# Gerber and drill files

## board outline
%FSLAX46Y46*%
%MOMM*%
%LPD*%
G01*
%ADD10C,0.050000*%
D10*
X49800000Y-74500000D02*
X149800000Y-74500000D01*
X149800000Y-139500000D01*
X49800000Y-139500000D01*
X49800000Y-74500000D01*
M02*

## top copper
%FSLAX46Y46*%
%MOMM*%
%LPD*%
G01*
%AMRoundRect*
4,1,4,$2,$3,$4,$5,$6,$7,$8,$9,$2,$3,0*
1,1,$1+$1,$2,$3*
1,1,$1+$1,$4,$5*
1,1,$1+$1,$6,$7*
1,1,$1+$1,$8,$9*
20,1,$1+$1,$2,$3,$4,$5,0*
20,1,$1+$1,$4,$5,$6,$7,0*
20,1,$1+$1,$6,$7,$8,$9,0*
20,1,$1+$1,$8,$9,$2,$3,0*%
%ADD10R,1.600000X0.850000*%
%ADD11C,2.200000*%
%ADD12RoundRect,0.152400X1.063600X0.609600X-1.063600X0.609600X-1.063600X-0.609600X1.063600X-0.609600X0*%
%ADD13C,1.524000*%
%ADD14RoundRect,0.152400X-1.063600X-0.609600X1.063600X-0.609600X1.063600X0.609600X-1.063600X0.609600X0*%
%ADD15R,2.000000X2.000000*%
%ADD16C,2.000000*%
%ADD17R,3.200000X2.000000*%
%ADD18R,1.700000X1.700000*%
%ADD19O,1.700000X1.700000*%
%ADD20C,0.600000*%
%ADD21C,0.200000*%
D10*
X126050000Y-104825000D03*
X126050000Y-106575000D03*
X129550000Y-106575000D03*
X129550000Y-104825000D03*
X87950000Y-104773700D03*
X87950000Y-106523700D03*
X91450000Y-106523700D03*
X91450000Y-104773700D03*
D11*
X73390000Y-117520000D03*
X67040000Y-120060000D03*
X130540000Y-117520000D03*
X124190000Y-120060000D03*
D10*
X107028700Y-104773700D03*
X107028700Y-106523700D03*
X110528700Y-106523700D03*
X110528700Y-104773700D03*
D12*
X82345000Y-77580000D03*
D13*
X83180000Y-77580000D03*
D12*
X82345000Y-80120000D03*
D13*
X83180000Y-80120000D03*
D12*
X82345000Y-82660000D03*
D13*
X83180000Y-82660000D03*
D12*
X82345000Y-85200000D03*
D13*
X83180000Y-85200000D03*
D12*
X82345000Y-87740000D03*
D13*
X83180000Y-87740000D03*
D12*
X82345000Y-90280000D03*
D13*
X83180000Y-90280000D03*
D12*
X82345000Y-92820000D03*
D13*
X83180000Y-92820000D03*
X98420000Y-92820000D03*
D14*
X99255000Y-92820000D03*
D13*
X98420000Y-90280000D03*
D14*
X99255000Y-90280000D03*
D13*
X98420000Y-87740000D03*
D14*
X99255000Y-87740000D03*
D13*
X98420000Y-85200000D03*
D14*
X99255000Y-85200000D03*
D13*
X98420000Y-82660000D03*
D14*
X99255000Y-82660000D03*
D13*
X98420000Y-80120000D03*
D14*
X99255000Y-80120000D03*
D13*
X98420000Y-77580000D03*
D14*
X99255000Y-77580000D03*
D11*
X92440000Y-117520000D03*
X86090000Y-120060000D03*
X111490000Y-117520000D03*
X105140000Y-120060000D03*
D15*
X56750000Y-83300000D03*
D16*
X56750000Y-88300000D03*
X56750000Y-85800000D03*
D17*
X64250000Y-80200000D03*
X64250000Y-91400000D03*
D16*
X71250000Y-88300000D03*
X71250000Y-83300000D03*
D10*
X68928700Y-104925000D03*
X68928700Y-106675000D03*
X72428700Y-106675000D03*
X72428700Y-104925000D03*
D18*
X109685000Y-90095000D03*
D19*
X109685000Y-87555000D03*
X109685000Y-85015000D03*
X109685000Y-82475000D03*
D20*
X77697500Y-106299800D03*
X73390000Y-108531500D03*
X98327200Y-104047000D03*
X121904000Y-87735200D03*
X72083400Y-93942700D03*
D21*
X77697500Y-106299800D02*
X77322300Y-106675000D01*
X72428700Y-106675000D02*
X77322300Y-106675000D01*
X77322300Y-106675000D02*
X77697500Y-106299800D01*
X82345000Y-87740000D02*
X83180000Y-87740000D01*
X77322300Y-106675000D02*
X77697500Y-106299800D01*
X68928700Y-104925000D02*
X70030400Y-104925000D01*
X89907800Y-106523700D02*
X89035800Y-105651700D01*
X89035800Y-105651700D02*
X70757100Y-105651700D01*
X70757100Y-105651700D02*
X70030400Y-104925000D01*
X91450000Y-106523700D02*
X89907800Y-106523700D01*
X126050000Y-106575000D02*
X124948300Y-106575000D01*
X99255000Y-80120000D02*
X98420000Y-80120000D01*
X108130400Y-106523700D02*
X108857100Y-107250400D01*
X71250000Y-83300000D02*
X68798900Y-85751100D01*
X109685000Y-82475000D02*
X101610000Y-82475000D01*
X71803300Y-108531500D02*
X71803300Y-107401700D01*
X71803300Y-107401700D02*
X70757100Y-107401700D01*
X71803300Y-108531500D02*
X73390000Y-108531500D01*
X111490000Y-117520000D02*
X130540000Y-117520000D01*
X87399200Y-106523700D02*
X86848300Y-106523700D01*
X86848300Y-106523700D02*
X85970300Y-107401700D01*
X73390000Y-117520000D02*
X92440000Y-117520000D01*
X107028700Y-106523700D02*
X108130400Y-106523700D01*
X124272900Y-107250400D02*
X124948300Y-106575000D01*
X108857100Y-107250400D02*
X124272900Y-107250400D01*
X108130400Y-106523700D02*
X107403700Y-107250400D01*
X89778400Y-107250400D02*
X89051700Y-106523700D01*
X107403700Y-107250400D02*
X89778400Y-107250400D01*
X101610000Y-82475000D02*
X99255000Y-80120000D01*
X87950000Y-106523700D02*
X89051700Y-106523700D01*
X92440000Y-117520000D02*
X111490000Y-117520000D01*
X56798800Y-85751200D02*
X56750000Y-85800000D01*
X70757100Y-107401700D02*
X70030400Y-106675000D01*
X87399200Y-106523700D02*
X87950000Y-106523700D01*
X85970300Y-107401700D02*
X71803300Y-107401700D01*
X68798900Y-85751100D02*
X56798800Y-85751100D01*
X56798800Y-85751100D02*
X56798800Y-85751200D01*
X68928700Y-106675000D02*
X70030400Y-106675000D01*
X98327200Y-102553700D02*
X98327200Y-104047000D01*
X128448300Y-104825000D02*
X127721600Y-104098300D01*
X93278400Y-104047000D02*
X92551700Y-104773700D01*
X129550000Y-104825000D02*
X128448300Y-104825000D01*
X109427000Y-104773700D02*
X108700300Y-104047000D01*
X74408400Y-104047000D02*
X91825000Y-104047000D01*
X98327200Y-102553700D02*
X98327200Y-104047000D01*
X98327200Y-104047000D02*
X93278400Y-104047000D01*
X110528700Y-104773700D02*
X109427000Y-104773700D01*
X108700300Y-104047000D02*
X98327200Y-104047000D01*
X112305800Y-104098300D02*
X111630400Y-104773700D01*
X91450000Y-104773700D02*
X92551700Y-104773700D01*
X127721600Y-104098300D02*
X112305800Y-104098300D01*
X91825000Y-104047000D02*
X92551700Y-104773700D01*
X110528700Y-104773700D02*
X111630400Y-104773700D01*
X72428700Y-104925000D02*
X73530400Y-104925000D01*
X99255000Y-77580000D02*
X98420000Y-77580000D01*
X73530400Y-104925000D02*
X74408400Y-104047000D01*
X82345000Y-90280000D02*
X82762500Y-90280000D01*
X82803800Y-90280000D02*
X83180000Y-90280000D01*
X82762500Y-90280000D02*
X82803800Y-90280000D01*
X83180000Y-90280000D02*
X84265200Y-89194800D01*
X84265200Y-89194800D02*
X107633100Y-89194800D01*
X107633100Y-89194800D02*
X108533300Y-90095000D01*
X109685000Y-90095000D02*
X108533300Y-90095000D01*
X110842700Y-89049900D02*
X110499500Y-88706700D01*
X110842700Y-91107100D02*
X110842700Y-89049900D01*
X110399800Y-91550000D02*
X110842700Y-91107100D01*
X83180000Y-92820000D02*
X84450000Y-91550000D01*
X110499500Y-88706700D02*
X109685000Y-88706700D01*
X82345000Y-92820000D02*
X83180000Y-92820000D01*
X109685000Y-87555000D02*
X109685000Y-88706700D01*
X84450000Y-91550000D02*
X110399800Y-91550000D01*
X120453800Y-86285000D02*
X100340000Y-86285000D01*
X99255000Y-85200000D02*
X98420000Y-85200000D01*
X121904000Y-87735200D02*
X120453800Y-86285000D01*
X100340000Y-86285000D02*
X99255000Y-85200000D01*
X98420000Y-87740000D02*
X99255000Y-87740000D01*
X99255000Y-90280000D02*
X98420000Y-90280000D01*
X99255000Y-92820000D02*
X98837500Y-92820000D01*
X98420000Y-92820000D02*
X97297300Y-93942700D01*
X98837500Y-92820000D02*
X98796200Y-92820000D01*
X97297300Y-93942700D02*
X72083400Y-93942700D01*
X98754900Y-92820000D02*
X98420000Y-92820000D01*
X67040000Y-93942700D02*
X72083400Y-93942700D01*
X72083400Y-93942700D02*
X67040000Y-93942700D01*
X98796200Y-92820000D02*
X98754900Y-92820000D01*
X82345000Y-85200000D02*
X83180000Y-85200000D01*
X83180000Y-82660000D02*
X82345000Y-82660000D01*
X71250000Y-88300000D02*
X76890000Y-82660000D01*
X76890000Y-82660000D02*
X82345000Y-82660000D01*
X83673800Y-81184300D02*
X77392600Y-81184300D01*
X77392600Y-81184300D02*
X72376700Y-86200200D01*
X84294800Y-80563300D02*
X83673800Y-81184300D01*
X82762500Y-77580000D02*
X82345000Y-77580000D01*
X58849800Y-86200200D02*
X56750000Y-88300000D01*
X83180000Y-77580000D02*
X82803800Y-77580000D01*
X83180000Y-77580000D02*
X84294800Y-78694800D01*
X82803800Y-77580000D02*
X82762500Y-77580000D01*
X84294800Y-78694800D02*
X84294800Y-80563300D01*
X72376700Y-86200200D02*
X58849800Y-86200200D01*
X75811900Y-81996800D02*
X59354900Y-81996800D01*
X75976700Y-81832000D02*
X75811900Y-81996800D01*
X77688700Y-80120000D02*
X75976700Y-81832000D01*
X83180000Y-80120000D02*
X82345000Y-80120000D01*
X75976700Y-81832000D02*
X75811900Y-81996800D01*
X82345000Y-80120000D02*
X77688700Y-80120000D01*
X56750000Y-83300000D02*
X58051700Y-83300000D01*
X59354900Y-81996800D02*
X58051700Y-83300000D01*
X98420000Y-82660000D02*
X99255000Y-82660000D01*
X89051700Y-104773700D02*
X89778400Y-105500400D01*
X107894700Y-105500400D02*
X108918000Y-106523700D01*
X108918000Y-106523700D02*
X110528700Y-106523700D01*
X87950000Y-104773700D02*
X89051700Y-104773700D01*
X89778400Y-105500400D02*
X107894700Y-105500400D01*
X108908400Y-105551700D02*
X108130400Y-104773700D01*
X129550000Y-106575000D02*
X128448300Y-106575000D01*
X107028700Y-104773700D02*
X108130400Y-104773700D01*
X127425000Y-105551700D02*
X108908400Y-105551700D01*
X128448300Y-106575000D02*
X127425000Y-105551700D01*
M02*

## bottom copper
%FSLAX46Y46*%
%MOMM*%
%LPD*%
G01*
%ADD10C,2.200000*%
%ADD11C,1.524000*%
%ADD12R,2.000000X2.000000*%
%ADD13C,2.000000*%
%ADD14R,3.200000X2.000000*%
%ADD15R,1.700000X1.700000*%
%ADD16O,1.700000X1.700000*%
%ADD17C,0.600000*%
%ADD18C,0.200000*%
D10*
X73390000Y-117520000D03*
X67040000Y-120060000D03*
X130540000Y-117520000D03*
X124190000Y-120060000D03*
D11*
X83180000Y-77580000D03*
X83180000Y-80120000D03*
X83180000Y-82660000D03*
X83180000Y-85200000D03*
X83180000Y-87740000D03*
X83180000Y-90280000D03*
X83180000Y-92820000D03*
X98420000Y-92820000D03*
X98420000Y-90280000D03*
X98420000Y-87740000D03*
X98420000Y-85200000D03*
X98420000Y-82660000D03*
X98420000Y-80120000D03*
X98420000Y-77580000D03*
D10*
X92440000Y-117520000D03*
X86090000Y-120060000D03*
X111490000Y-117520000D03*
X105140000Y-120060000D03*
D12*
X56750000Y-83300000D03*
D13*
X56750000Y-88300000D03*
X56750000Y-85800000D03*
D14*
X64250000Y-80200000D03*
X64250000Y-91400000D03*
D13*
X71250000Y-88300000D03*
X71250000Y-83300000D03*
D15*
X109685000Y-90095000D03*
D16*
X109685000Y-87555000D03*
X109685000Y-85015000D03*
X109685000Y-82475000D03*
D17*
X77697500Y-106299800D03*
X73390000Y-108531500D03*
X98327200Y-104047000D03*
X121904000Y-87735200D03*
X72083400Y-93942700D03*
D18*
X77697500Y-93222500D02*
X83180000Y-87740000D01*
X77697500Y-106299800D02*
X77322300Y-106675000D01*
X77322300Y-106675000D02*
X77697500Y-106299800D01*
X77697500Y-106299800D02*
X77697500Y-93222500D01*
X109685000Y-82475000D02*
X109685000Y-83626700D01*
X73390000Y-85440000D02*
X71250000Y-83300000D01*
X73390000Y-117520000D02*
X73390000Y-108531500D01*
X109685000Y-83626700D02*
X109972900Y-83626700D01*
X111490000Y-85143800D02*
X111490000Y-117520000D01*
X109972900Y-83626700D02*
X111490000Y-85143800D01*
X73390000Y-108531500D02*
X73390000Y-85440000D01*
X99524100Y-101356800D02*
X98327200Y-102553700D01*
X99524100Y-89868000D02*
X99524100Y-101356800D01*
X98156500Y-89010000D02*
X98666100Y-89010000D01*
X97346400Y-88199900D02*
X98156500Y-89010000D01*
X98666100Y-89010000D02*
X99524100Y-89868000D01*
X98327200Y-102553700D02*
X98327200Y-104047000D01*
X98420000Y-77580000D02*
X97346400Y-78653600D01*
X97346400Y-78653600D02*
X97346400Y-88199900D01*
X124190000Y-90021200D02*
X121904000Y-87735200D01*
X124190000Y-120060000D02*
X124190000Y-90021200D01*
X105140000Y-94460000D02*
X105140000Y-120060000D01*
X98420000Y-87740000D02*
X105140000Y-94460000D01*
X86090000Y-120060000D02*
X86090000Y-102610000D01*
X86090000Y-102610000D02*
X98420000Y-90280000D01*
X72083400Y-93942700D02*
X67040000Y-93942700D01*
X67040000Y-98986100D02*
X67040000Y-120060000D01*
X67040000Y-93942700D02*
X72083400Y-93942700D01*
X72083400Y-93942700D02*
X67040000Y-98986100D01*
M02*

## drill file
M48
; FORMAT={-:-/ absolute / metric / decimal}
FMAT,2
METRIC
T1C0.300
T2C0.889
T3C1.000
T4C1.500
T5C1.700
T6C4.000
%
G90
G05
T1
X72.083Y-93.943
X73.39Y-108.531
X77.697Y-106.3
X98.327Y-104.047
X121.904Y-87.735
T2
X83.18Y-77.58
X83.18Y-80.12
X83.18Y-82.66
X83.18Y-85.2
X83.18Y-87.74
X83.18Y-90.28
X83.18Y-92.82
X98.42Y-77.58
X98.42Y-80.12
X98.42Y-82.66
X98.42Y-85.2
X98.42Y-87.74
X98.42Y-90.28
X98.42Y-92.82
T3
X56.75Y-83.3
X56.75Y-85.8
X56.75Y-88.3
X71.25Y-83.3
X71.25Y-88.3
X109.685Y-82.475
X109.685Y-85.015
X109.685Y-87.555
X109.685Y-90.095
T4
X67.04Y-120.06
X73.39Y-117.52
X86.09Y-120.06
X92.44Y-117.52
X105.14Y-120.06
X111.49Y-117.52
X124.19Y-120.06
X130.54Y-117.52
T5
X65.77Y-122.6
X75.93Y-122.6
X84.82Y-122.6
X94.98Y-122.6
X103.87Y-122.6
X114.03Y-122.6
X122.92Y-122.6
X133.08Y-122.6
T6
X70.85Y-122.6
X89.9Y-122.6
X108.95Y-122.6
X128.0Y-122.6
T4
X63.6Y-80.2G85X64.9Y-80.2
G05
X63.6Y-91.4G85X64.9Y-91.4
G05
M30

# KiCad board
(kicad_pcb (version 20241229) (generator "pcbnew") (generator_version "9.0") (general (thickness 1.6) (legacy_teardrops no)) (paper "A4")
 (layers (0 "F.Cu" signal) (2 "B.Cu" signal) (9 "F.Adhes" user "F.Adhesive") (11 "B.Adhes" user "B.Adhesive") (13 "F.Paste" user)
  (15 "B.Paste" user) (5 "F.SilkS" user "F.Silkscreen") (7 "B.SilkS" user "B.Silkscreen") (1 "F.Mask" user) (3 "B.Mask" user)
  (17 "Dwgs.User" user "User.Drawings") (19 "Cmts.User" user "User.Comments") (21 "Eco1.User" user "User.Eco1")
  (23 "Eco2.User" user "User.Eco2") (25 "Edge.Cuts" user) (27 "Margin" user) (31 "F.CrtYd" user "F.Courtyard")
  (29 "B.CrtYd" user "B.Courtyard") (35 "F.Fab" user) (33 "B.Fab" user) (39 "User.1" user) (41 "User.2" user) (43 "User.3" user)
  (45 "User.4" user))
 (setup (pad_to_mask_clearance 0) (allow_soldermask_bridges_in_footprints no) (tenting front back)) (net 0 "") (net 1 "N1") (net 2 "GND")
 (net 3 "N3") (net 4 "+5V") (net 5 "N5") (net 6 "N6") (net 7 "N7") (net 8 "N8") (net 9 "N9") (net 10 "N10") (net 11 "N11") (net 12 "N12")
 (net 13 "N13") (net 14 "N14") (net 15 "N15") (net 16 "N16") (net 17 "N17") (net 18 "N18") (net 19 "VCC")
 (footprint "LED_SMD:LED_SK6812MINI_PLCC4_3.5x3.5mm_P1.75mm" (layer "F.Cu") (at 127.8 105.7)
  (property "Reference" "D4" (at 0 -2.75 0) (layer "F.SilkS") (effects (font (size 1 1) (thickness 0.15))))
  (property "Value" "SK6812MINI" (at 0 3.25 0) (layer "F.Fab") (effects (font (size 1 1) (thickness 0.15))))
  (pad "1" smd rect (at -1.75 -0.875) (size 1.6 0.85) (layers "F.Cu" "F.Mask" "F.Paste") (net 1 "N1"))
  (pad "2" smd rect (at -1.75 0.875) (size 1.6 0.85) (layers "F.Cu" "F.Mask" "F.Paste") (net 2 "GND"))
  (pad "3" smd rect (at 1.75 0.875) (size 1.6 0.85) (layers "F.Cu" "F.Mask" "F.Paste") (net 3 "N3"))
  (pad "4" smd rect (at 1.75 -0.875) (size 1.6 0.85) (layers "F.Cu" "F.Mask" "F.Paste") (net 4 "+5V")))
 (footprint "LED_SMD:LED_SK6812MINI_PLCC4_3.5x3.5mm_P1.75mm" (layer "F.Cu") (at 89.7 105.6487)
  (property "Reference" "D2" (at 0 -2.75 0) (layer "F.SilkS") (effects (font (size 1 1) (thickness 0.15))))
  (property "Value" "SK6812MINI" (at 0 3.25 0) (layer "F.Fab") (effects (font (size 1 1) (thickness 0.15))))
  (pad "1" smd rect (at -1.75 -0.875) (size 1.6 0.85) (layers "F.Cu" "F.Mask" "F.Paste") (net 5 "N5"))
  (pad "2" smd rect (at -1.75 0.875) (size 1.6 0.85) (layers "F.Cu" "F.Mask" "F.Paste") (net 2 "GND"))
  (pad "3" smd rect (at 1.75 0.875) (size 1.6 0.85) (layers "F.Cu" "F.Mask" "F.Paste") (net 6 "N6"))
  (pad "4" smd rect (at 1.75 -0.875) (size 1.6 0.85) (layers "F.Cu" "F.Mask" "F.Paste") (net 4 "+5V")))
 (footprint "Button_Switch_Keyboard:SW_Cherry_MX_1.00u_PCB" (layer "F.Cu") (at 73.39 117.52)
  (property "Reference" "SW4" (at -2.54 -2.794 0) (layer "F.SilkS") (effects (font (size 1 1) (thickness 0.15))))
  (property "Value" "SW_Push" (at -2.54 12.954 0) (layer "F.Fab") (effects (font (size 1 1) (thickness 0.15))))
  (pad "" np_thru_hole circle (at -7.62 5.08) (size 1.7 1.7) (drill 1.7) (layers "*.Cu" "*.Mask"))
  (pad "" np_thru_hole circle (at -2.54 5.08) (size 4 4) (drill 4) (layers "*.Cu" "*.Mask"))
  (pad "" np_thru_hole circle (at 2.54 5.08) (size 1.7 1.7) (drill 1.7) (layers "*.Cu" "*.Mask"))
  (pad "1" thru_hole circle (at 0 0) (size 2.2 2.2) (drill 1.5) (layers "*.Cu" "*.Mask") (remove_unused_layers no) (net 2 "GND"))
  (pad "2" thru_hole circle (at -6.35 2.54) (size 2.2 2.2) (drill 1.5) (layers "*.Cu" "*.Mask") (remove_unused_layers no) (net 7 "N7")))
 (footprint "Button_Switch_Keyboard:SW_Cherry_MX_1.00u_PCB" (layer "F.Cu") (at 130.54 117.52)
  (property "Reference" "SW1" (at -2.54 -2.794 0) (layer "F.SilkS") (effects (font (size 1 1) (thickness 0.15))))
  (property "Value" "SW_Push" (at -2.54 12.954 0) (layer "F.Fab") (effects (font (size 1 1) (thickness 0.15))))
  (pad "" np_thru_hole circle (at -7.62 5.08) (size 1.7 1.7) (drill 1.7) (layers "*.Cu" "*.Mask"))
  (pad "" np_thru_hole circle (at -2.54 5.08) (size 4 4) (drill 4) (layers "*.Cu" "*.Mask"))
  (pad "" np_thru_hole circle (at 2.54 5.08) (size 1.7 1.7) (drill 1.7) (layers "*.Cu" "*.Mask"))
  (pad "1" thru_hole circle (at 0 0) (size 2.2 2.2) (drill 1.5) (layers "*.Cu" "*.Mask") (remove_unused_layers no) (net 2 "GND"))
  (pad "2" thru_hole circle (at -6.35 2.54) (size 2.2 2.2) (drill 1.5) (layers "*.Cu" "*.Mask") (remove_unused_layers no) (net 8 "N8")))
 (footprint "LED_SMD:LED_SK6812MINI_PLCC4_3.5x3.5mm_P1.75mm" (layer "F.Cu") (at 108.7787 105.6487)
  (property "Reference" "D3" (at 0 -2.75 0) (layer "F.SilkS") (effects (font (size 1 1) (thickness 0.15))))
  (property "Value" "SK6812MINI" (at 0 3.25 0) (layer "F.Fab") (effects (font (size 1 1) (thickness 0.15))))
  (pad "1" smd rect (at -1.75 -0.875) (size 1.6 0.85) (layers "F.Cu" "F.Mask" "F.Paste") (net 3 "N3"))
  (pad "2" smd rect (at -1.75 0.875) (size 1.6 0.85) (layers "F.Cu" "F.Mask" "F.Paste") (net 2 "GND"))
  (pad "3" smd rect (at 1.75 0.875) (size 1.6 0.85) (layers "F.Cu" "F.Mask" "F.Paste") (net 5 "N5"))
  (pad "4" smd rect (at 1.75 -0.875) (size 1.6 0.85) (layers "F.Cu" "F.Mask" "F.Paste") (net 4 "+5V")))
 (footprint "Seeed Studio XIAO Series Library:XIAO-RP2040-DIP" (layer "F.Cu") (at 90.8 85.2)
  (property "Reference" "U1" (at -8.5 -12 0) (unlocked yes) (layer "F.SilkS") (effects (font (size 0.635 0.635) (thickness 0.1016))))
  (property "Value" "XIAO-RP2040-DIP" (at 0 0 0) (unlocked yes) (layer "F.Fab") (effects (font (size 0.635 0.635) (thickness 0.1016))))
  (pad "1" smd roundrect (at -8.455 -7.62 180) (size 2.432 1.524) (layers "F.Cu" "F.Mask") (roundrect_rratio 0.1) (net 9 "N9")
   (thermal_bridge_angle 45))
  (pad "1" thru_hole circle (at -7.62 -7.62 180) (size 1.524 1.524) (drill 0.889) (layers "*.Cu" "*.Mask") (remove_unused_layers no)
   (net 9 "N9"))
  (pad "2" smd roundrect (at -8.455 -5.08 180) (size 2.432 1.524) (layers "F.Cu" "F.Mask") (roundrect_rratio 0.1) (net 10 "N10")
   (thermal_bridge_angle 45))
  (pad "2" thru_hole circle (at -7.62 -5.08 180) (size 1.524 1.524) (drill 0.889) (layers "*.Cu" "*.Mask") (remove_unused_layers no)
   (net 10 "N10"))
  (pad "3" smd roundrect (at -8.455 -2.54 180) (size 2.432 1.524) (layers "F.Cu" "F.Mask") (roundrect_rratio 0.1) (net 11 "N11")
   (thermal_bridge_angle 45))
  (pad "3" thru_hole circle (at -7.62 -2.54 180) (size 1.524 1.524) (drill 0.889) (layers "*.Cu" "*.Mask") (remove_unused_layers no)
   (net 11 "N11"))
  (pad "4" smd roundrect (at -8.455 0 180) (size 2.432 1.524) (layers "F.Cu" "F.Mask") (roundrect_rratio 0.1) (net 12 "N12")
   (thermal_bridge_angle 45))
  (pad "4" thru_hole circle (at -7.62 0 180) (size 1.524 1.524) (drill 0.889) (layers "*.Cu" "*.Mask") (remove_unused_layers no)
   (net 12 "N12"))
  (pad "5" smd roundrect (at -8.455 2.54 180) (size 2.432 1.524) (layers "F.Cu" "F.Mask") (roundrect_rratio 0.1) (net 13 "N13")
   (thermal_bridge_angle 45))
  (pad "5" thru_hole circle (at -7.62 2.54 180) (size 1.524 1.524) (drill 0.889) (layers "*.Cu" "*.Mask") (remove_unused_layers no)
   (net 13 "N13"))
  (pad "6" smd roundrect (at -8.455 5.08 180) (size 2.432 1.524) (layers "F.Cu" "F.Mask") (roundrect_rratio 0.1) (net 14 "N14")
   (thermal_bridge_angle 45))
  (pad "6" thru_hole circle (at -7.62 5.08 180) (size 1.524 1.524) (drill 0.889) (layers "*.Cu" "*.Mask") (remove_unused_layers no)
   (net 14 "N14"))
  (pad "7" smd roundrect (at -8.455 7.62 180) (size 2.432 1.524) (layers "F.Cu" "F.Mask") (roundrect_rratio 0.1) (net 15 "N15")
   (thermal_bridge_angle 45))
  (pad "7" thru_hole circle (at -7.62 7.62 180) (size 1.524 1.524) (drill 0.889) (layers "*.Cu" "*.Mask") (remove_unused_layers no)
   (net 15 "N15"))
  (pad "8" thru_hole circle (at 7.62 7.62) (size 1.524 1.524) (drill 0.889) (layers "*.Cu" "*.Mask") (remove_unused_layers no) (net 7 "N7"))
  (pad "8" smd roundrect (at 8.455 7.62) (size 2.432 1.524) (layers "F.Cu" "F.Mask") (roundrect_rratio 0.1) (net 7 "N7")
   (thermal_bridge_angle 45))
  (pad "9" thru_hole circle (at 7.62 5.08) (size 1.524 1.524) (drill 0.889) (layers "*.Cu" "*.Mask") (remove_unused_layers no)
   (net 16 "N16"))
  (pad "9" smd roundrect (at 8.455 5.08) (size 2.432 1.524) (layers "F.Cu" "F.Mask") (roundrect_rratio 0.1) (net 16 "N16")
   (thermal_bridge_angle 45))
  (pad "10" thru_hole circle (at 7.62 2.54) (size 1.524 1.524) (drill 0.889) (layers "*.Cu" "*.Mask") (remove_unused_layers no)
   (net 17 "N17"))
  (pad "10" smd roundrect (at 8.455 2.54) (size 2.432 1.524) (layers "F.Cu" "F.Mask") (roundrect_rratio 0.1) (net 17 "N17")
   (thermal_bridge_angle 45))
  (pad "11" thru_hole circle (at 7.62 0) (size 1.524 1.524) (drill 0.889) (layers "*.Cu" "*.Mask") (remove_unused_layers no) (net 8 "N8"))
  (pad "11" smd roundrect (at 8.455 0) (size 2.432 1.524) (layers "F.Cu" "F.Mask") (roundrect_rratio 0.1) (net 8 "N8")
   (thermal_bridge_angle 45))
  (pad "12" thru_hole circle (at 7.62 -2.54) (size 1.524 1.524) (drill 0.889) (layers "*.Cu" "*.Mask") (remove_unused_layers no)
   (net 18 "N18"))
  (pad "12" smd roundrect (at 8.455 -2.54) (size 2.432 1.524) (layers "F.Cu" "F.Mask") (roundrect_rratio 0.1) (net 18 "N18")
   (thermal_bridge_angle 45))
  (pad "13" thru_hole circle (at 7.62 -5.08) (size 1.524 1.524) (drill 0.889) (layers "*.Cu" "*.Mask") (remove_unused_layers no)
   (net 2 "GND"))
  (pad "13" smd roundrect (at 8.455 -5.08) (size 2.432 1.524) (layers "F.Cu" "F.Mask") (roundrect_rratio 0.1) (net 2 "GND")
   (thermal_bridge_angle 45))
  (pad "14" thru_hole circle (at 7.62 -7.62) (size 1.524 1.524) (drill 0.889) (layers "*.Cu" "*.Mask") (remove_unused_layers no)
   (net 4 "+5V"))
  (pad "14" smd roundrect (at 8.455 -7.62) (size 2.432 1.524) (layers "F.Cu" "F.Mask") (roundrect_rratio 0.1) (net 4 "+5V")
   (thermal_bridge_angle 45)))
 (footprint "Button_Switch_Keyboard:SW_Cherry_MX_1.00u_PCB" (layer "F.Cu") (at 92.44 117.52)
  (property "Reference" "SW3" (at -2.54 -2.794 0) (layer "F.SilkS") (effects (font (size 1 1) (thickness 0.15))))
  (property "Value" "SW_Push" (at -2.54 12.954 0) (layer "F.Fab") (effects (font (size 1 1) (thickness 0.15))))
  (pad "" np_thru_hole circle (at -7.62 5.08) (size 1.7 1.7) (drill 1.7) (layers "*.Cu" "*.Mask"))
  (pad "" np_thru_hole circle (at -2.54 5.08) (size 4 4) (drill 4) (layers "*.Cu" "*.Mask"))
  (pad "" np_thru_hole circle (at 2.54 5.08) (size 1.7 1.7) (drill 1.7) (layers "*.Cu" "*.Mask"))
  (pad "1" thru_hole circle (at 0 0) (size 2.2 2.2) (drill 1.5) (layers "*.Cu" "*.Mask") (remove_unused_layers no) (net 2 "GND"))
  (pad "2" thru_hole circle (at -6.35 2.54) (size 2.2 2.2) (drill 1.5) (layers "*.Cu" "*.Mask") (remove_unused_layers no) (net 16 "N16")))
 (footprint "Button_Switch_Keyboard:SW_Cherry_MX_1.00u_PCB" (layer "F.Cu") (at 111.49 117.52)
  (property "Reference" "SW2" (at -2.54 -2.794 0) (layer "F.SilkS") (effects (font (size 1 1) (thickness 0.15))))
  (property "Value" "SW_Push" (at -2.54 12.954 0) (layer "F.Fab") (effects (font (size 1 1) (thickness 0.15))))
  (pad "" np_thru_hole circle (at -7.62 5.08) (size 1.7 1.7) (drill 1.7) (layers "*.Cu" "*.Mask"))
  (pad "" np_thru_hole circle (at -2.54 5.08) (size 4 4) (drill 4) (layers "*.Cu" "*.Mask"))
  (pad "" np_thru_hole circle (at 2.54 5.08) (size 1.7 1.7) (drill 1.7) (layers "*.Cu" "*.Mask"))
  (pad "1" thru_hole circle (at 0 0) (size 2.2 2.2) (drill 1.5) (layers "*.Cu" "*.Mask") (remove_unused_layers no) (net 2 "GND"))
  (pad "2" thru_hole circle (at -6.35 2.54) (size 2.2 2.2) (drill 1.5) (layers "*.Cu" "*.Mask") (remove_unused_layers no) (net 17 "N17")))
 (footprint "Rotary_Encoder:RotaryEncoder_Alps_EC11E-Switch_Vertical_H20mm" (layer "F.Cu") (at 56.75 83.3)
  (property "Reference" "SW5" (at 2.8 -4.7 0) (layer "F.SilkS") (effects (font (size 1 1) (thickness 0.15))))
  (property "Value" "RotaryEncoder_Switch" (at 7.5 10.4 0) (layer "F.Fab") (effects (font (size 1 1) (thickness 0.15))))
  (pad "A" thru_hole rect (at 0 0) (size 2 2) (drill 1) (layers "*.Cu" "*.Mask") (remove_unused_layers no) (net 10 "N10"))
  (pad "B" thru_hole circle (at 0 5) (size 2 2) (drill 1) (layers "*.Cu" "*.Mask") (remove_unused_layers no) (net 9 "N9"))
  (pad "C" thru_hole circle (at 0 2.5) (size 2 2) (drill 1) (layers "*.Cu" "*.Mask") (remove_unused_layers no) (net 2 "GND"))
  (pad "MP" thru_hole rect (at 7.5 -3.1) (size 3.2 2) (drill oval 2.8 1.5) (layers "*.Cu" "*.Mask") (remove_unused_layers no))
  (pad "MP" thru_hole rect (at 7.5 8.1) (size 3.2 2) (drill oval 2.8 1.5) (layers "*.Cu" "*.Mask") (remove_unused_layers no))
  (pad "S1" thru_hole circle (at 14.5 5) (size 2 2) (drill 1) (layers "*.Cu" "*.Mask") (remove_unused_layers no) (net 11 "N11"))
  (pad "S2" thru_hole circle (at 14.5 0) (size 2 2) (drill 1) (layers "*.Cu" "*.Mask") (remove_unused_layers no) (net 2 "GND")))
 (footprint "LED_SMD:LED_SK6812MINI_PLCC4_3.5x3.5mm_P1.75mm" (layer "F.Cu") (at 70.6787 105.8)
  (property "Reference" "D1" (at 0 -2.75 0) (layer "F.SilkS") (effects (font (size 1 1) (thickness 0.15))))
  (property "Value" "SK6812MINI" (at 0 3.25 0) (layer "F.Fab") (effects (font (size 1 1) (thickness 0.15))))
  (pad "1" smd rect (at -1.75 -0.875) (size 1.6 0.85) (layers "F.Cu" "F.Mask" "F.Paste") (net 6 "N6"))
  (pad "2" smd rect (at -1.75 0.875) (size 1.6 0.85) (layers "F.Cu" "F.Mask" "F.Paste") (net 2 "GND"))
  (pad "3" smd rect (at 1.75 0.875) (size 1.6 0.85) (layers "F.Cu" "F.Mask" "F.Paste") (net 13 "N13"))
  (pad "4" smd rect (at 1.75 -0.875) (size 1.6 0.85) (layers "F.Cu" "F.Mask" "F.Paste") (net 4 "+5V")))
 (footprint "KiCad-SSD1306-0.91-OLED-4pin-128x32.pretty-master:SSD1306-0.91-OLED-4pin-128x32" (layer "F.Cu") (at 146.185 92.285 180)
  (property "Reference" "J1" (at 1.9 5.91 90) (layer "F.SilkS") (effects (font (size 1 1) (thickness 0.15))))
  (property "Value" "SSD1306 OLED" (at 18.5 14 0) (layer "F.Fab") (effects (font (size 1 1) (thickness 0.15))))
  (pad "1" thru_hole rect (at 36.5 2.19 180) (size 1.7 1.7) (drill 1) (layers "*.Cu" "*.Mask") (remove_unused_layers no) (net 14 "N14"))
  (pad "2" thru_hole oval (at 36.5 4.73 180) (size 1.7 1.7) (drill 1) (layers "*.Cu" "*.Mask") (remove_unused_layers no) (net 15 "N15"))
  (pad "3" thru_hole oval (at 36.5 7.27 180) (size 1.7 1.7) (drill 1) (layers "*.Cu" "*.Mask") (remove_unused_layers no) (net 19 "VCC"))
  (pad "4" thru_hole oval (at 36.5 9.81 180) (size 1.7 1.7) (drill 1) (layers "*.Cu" "*.Mask") (remove_unused_layers no) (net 2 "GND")))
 (gr_rect (start 49.8 74.5) (end 149.8 139.5) (stroke (width 0.05) (type default)) (fill no) (layer "Edge.Cuts"))
 (segment (start 77.6975 106.2998) (end 77.3223 106.675) (width 0.2) (layer "F.Cu") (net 13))
 (segment (start 72.4287 106.675) (end 77.3223 106.675) (width 0.2) (layer "F.Cu") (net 13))
 (segment (start 77.3223 106.675) (end 77.6975 106.2998) (width 0.2) (layer "F.Cu") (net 13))
 (segment (start 82.345 87.74) (end 83.18 87.74) (width 0.2) (layer "F.Cu") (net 13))
 (segment (start 77.3223 106.675) (end 77.6975 106.2998) (width 0.2) (layer "F.Cu") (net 13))
 (via (at 77.6975 106.2998) (size 0.6) (drill 0.3) (layers "F.Cu" "B.Cu") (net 13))
 (segment (start 77.6975 93.2225) (end 83.18 87.74) (width 0.2) (layer "B.Cu") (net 13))
 (segment (start 77.6975 106.2998) (end 77.3223 106.675) (width 0.2) (layer "B.Cu") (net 13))
 (segment (start 77.3223 106.675) (end 77.6975 106.2998) (width 0.2) (layer "B.Cu") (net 13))
 (segment (start 77.6975 106.2998) (end 77.6975 93.2225) (width 0.2) (layer "B.Cu") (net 13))
 (segment (start 68.9287 104.925) (end 70.0304 104.925) (width 0.2) (layer "F.Cu") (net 6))
 (segment (start 89.9078 106.5237) (end 89.0358 105.6517) (width 0.2) (layer "F.Cu") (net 6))
 (segment (start 89.0358 105.6517) (end 70.7571 105.6517) (width 0.2) (layer "F.Cu") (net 6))
 (segment (start 70.7571 105.6517) (end 70.0304 104.925) (width 0.2) (layer "F.Cu") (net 6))
 (segment (start 91.45 106.5237) (end 89.9078 106.5237) (width 0.2) (layer "F.Cu") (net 6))
 (segment (start 126.05 106.575) (end 124.9483 106.575) (width 0.2) (layer "F.Cu") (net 2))
 (segment (start 99.255 80.12) (end 98.42 80.12) (width 0.2) (layer "F.Cu") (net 2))
 (segment (start 108.1304 106.5237) (end 108.8571 107.2504) (width 0.2) (layer "F.Cu") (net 2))
 (segment (start 71.25 83.3) (end 68.7989 85.7511) (width 0.2) (layer "F.Cu") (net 2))
 (segment (start 109.685 82.475) (end 101.61 82.475) (width 0.2) (layer "F.Cu") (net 2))
 (segment (start 71.8033 108.5315) (end 71.8033 107.4017) (width 0.2) (layer "F.Cu") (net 2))
 (segment (start 71.8033 107.4017) (end 70.7571 107.4017) (width 0.2) (layer "F.Cu") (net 2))
 (segment (start 71.8033 108.5315) (end 73.39 108.5315) (width 0.2) (layer "F.Cu") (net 2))
 (segment (start 111.49 117.52) (end 130.54 117.52) (width 0.2) (layer "F.Cu") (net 2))
 (segment (start 87.3992 106.5237) (end 86.8483 106.5237) (width 0.2) (layer "F.Cu") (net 2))
 (segment (start 86.8483 106.5237) (end 85.9703 107.4017) (width 0.2) (layer "F.Cu") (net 2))
 (segment (start 73.39 117.52) (end 92.44 117.52) (width 0.2) (layer "F.Cu") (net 2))
 (segment (start 107.0287 106.5237) (end 108.1304 106.5237) (width 0.2) (layer "F.Cu") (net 2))
 (segment (start 124.2729 107.2504) (end 124.9483 106.575) (width 0.2) (layer "F.Cu") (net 2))
 (segment (start 108.8571 107.2504) (end 124.2729 107.2504) (width 0.2) (layer "F.Cu") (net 2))
 (segment (start 108.1304 106.5237) (end 107.4037 107.2504) (width 0.2) (layer "F.Cu") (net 2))
 (segment (start 89.7784 107.2504) (end 89.0517 106.5237) (width 0.2) (layer "F.Cu") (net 2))
 (segment (start 107.4037 107.2504) (end 89.7784 107.2504) (width 0.2) (layer "F.Cu") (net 2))
 (segment (start 101.61 82.475) (end 99.255 80.12) (width 0.2) (layer "F.Cu") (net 2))
 (segment (start 87.95 106.5237) (end 89.0517 106.5237) (width 0.2) (layer "F.Cu") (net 2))
 (segment (start 92.44 117.52) (end 111.49 117.52) (width 0.2) (layer "F.Cu") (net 2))
 (segment (start 56.7988 85.7512) (end 56.75 85.8) (width 0.2) (layer "F.Cu") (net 2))
 (segment (start 70.7571 107.4017) (end 70.0304 106.675) (width 0.2) (layer "F.Cu") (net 2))
 (segment (start 87.3992 106.5237) (end 87.95 106.5237) (width 0.2) (layer "F.Cu") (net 2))
 (segment (start 85.9703 107.4017) (end 71.8033 107.4017) (width 0.2) (layer "F.Cu") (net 2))
 (segment (start 68.7989 85.7511) (end 56.7988 85.7511) (width 0.2) (layer "F.Cu") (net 2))
 (segment (start 56.7988 85.7511) (end 56.7988 85.7512) (width 0.2) (layer "F.Cu") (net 2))
 (segment (start 68.9287 106.675) (end 70.0304 106.675) (width 0.2) (layer "F.Cu") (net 2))
 (via (at 73.39 108.5315) (size 0.6) (drill 0.3) (layers "F.Cu" "B.Cu") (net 2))
 (segment (start 109.685 82.475) (end 109.685 83.6267) (width 0.2) (layer "B.Cu") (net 2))
 (segment (start 73.39 85.44) (end 71.25 83.3) (width 0.2) (layer "B.Cu") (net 2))
 (segment (start 73.39 117.52) (end 73.39 108.5315) (width 0.2) (layer "B.Cu") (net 2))
 (segment (start 109.685 83.6267) (end 109.9729 83.6267) (width 0.2) (layer "B.Cu") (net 2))
 (segment (start 111.49 85.1438) (end 111.49 117.52) (width 0.2) (layer "B.Cu") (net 2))
 (segment (start 109.9729 83.6267) (end 111.49 85.1438) (width 0.2) (layer "B.Cu") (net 2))
 (segment (start 73.39 108.5315) (end 73.39 85.44) (width 0.2) (layer "B.Cu") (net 2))
 (segment (start 98.3272 102.5537) (end 98.3272 104.047) (width 0.2) (layer "F.Cu") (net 4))
 (segment (start 128.4483 104.825) (end 127.7216 104.0983) (width 0.2) (layer "F.Cu") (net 4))
 (segment (start 93.2784 104.047) (end 92.5517 104.7737) (width 0.2) (layer "F.Cu") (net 4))
 (segment (start 129.55 104.825) (end 128.4483 104.825) (width 0.2) (layer "F.Cu") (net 4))
 (segment (start 109.427 104.7737) (end 108.7003 104.047) (width 0.2) (layer "F.Cu") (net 4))
 (segment (start 74.4084 104.047) (end 91.825 104.047) (width 0.2) (layer "F.Cu") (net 4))
 (segment (start 98.3272 102.5537) (end 98.3272 104.047) (width 0.2) (layer "F.Cu") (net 4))
 (segment (start 98.3272 104.047) (end 93.2784 104.047) (width 0.2) (layer "F.Cu") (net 4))
 (segment (start 110.5287 104.7737) (end 109.427 104.7737) (width 0.2) (layer "F.Cu") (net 4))
 (segment (start 108.7003 104.047) (end 98.3272 104.047) (width 0.2) (layer "F.Cu") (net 4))
 (segment (start 112.3058 104.0983) (end 111.6304 104.7737) (width 0.2) (layer "F.Cu") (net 4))
 (segment (start 91.45 104.7737) (end 92.5517 104.7737) (width 0.2) (layer "F.Cu") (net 4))
 (segment (start 127.7216 104.0983) (end 112.3058 104.0983) (width 0.2) (layer "F.Cu") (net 4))
 (segment (start 91.825 104.047) (end 92.5517 104.7737) (width 0.2) (layer "F.Cu") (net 4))
 (segment (start 110.5287 104.7737) (end 111.6304 104.7737) (width 0.2) (layer "F.Cu") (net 4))
 (segment (start 72.4287 104.925) (end 73.5304 104.925) (width 0.2) (layer "F.Cu") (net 4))
 (segment (start 99.255 77.58) (end 98.42 77.58) (width 0.2) (layer "F.Cu") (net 4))
 (segment (start 73.5304 104.925) (end 74.4084 104.047) (width 0.2) (layer "F.Cu") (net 4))
 (via (at 98.3272 104.047) (size 0.6) (drill 0.3) (layers "F.Cu" "B.Cu") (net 4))
 (segment (start 99.5241 101.3568) (end 98.3272 102.5537) (width 0.2) (layer "B.Cu") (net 4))
 (segment (start 99.5241 89.868) (end 99.5241 101.3568) (width 0.2) (layer "B.Cu") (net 4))
 (segment (start 98.1565 89.01) (end 98.6661 89.01) (width 0.2) (layer "B.Cu") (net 4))
 (segment (start 97.3464 88.1999) (end 98.1565 89.01) (width 0.2) (layer "B.Cu") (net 4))
 (segment (start 98.6661 89.01) (end 99.5241 89.868) (width 0.2) (layer "B.Cu") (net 4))
 (segment (start 98.3272 102.5537) (end 98.3272 104.047) (width 0.2) (layer "B.Cu") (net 4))
 (segment (start 98.42 77.58) (end 97.3464 78.6536) (width 0.2) (layer "B.Cu") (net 4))
 (segment (start 97.3464 78.6536) (end 97.3464 88.1999) (width 0.2) (layer "B.Cu") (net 4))
 (segment (start 82.345 90.28) (end 82.7625 90.28) (width 0.2) (layer "F.Cu") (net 14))
 (segment (start 82.8038 90.28) (end 83.18 90.28) (width 0.2) (layer "F.Cu") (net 14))
 (segment (start 82.7625 90.28) (end 82.8038 90.28) (width 0.2) (layer "F.Cu") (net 14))
 (segment (start 83.18 90.28) (end 84.2652 89.1948) (width 0.2) (layer "F.Cu") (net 14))
 (segment (start 84.2652 89.1948) (end 107.6331 89.1948) (width 0.2) (layer "F.Cu") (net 14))
 (segment (start 107.6331 89.1948) (end 108.5333 90.095) (width 0.2) (layer "F.Cu") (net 14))
 (segment (start 109.685 90.095) (end 108.5333 90.095) (width 0.2) (layer "F.Cu") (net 14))
 (segment (start 110.8427 89.0499) (end 110.4995 88.7067) (width 0.2) (layer "F.Cu") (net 15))
 (segment (start 110.8427 91.1071) (end 110.8427 89.0499) (width 0.2) (layer "F.Cu") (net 15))
 (segment (start 110.3998 91.55) (end 110.8427 91.1071) (width 0.2) (layer "F.Cu") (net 15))
 (segment (start 83.18 92.82) (end 84.45 91.55) (width 0.2) (layer "F.Cu") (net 15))
 (segment (start 110.4995 88.7067) (end 109.685 88.7067) (width 0.2) (layer "F.Cu") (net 15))
 (segment (start 82.345 92.82) (end 83.18 92.82) (width 0.2) (layer "F.Cu") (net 15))
 (segment (start 109.685 87.555) (end 109.685 88.7067) (width 0.2) (layer "F.Cu") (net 15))
 (segment (start 84.45 91.55) (end 110.3998 91.55) (width 0.2) (layer "F.Cu") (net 15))
 (segment (start 120.4538 86.285) (end 100.34 86.285) (width 0.2) (layer "F.Cu") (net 8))
 (segment (start 99.255 85.2) (end 98.42 85.2) (width 0.2) (layer "F.Cu") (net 8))
 (segment (start 121.904 87.7352) (end 120.4538 86.285) (width 0.2) (layer "F.Cu") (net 8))
 (segment (start 100.34 86.285) (end 99.255 85.2) (width 0.2) (layer "F.Cu") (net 8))
 (via (at 121.904 87.7352) (size 0.6) (drill 0.3) (layers "F.Cu" "B.Cu") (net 8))
 (segment (start 124.19 90.0212) (end 121.904 87.7352) (width 0.2) (layer "B.Cu") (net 8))
 (segment (start 124.19 120.06) (end 124.19 90.0212) (width 0.2) (layer "B.Cu") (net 8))
 (segment (start 98.42 87.74) (end 99.255 87.74) (width 0.2) (layer "F.Cu") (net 17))
 (segment (start 105.14 94.46) (end 105.14 120.06) (width 0.2) (layer "B.Cu") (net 17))
 (segment (start 98.42 87.74) (end 105.14 94.46) (width 0.2) (layer "B.Cu") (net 17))
 (segment (start 99.255 90.28) (end 98.42 90.28) (width 0.2) (layer "F.Cu") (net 16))
 (segment (start 86.09 120.06) (end 86.09 102.61) (width 0.2) (layer "B.Cu") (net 16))
 (segment (start 86.09 102.61) (end 98.42 90.28) (width 0.2) (layer "B.Cu") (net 16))
 (segment (start 99.255 92.82) (end 98.8375 92.82) (width 0.2) (layer "F.Cu") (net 7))
 (segment (start 98.42 92.82) (end 97.2973 93.9427) (width 0.2) (layer "F.Cu") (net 7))
 (segment (start 98.8375 92.82) (end 98.7962 92.82) (width 0.2) (layer "F.Cu") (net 7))
 (segment (start 97.2973 93.9427) (end 72.0834 93.9427) (width 0.2) (layer "F.Cu") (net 7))
 (segment (start 98.7549 92.82) (end 98.42 92.82) (width 0.2) (layer "F.Cu") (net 7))
 (segment (start 67.04 93.9427) (end 72.0834 93.9427) (width 0.2) (layer "F.Cu") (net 7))
 (segment (start 72.0834 93.9427) (end 67.04 93.9427) (width 0.2) (layer "F.Cu") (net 7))
 (segment (start 98.7962 92.82) (end 98.7549 92.82) (width 0.2) (layer "F.Cu") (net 7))
 (via (at 72.0834 93.9427) (size 0.6) (drill 0.3) (layers "F.Cu" "B.Cu") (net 7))
 (segment (start 72.0834 93.9427) (end 67.04 93.9427) (width 0.2) (layer "B.Cu") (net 7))
 (segment (start 67.04 98.9861) (end 67.04 120.06) (width 0.2) (layer "B.Cu") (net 7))
 (segment (start 67.04 93.9427) (end 72.0834 93.9427) (width 0.2) (layer "B.Cu") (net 7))
 (segment (start 72.0834 93.9427) (end 67.04 98.9861) (width 0.2) (layer "B.Cu") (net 7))
 (segment (start 82.345 85.2) (end 83.18 85.2) (width 0.2) (layer "F.Cu") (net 12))
 (segment (start 83.18 82.66) (end 82.345 82.66) (width 0.2) (layer "F.Cu") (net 11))
 (segment (start 71.25 88.3) (end 76.89 82.66) (width 0.2) (layer "F.Cu") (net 11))
 (segment (start 76.89 82.66) (end 82.345 82.66) (width 0.2) (layer "F.Cu") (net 11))
 (segment (start 83.6738 81.1843) (end 77.3926 81.1843) (width 0.2) (layer "F.Cu") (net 9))
 (segment (start 77.3926 81.1843) (end 72.3767 86.2002) (width 0.2) (layer "F.Cu") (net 9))
 (segment (start 84.2948 80.5633) (end 83.6738 81.1843) (width 0.2) (layer "F.Cu") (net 9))
 (segment (start 82.7625 77.58) (end 82.345 77.58) (width 0.2) (layer "F.Cu") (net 9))
 (segment (start 58.8498 86.2002) (end 56.75 88.3) (width 0.2) (layer "F.Cu") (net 9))
 (segment (start 83.18 77.58) (end 82.8038 77.58) (width 0.2) (layer "F.Cu") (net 9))
 (segment (start 83.18 77.58) (end 84.2948 78.6948) (width 0.2) (layer "F.Cu") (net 9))
 (segment (start 82.8038 77.58) (end 82.7625 77.58) (width 0.2) (layer "F.Cu") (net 9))
 (segment (start 84.2948 78.6948) (end 84.2948 80.5633) (width 0.2) (layer "F.Cu") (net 9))
 (segment (start 72.3767 86.2002) (end 58.8498 86.2002) (width 0.2) (layer "F.Cu") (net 9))
 (segment (start 75.8119 81.9968) (end 59.3549 81.9968) (width 0.2) (layer "F.Cu") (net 10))
 (segment (start 75.9767 81.832) (end 75.8119 81.9968) (width 0.2) (layer "F.Cu") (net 10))
 (segment (start 77.6887 80.12) (end 75.9767 81.832) (width 0.2) (layer "F.Cu") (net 10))
 (segment (start 83.18 80.12) (end 82.345 80.12) (width 0.2) (layer "F.Cu") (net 10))
 (segment (start 75.9767 81.832) (end 75.8119 81.9968) (width 0.2) (layer "F.Cu") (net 10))
 (segment (start 82.345 80.12) (end 77.6887 80.12) (width 0.2) (layer "F.Cu") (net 10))
 (segment (start 56.75 83.3) (end 58.0517 83.3) (width 0.2) (layer "F.Cu") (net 10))
 (segment (start 59.3549 81.9968) (end 58.0517 83.3) (width 0.2) (layer "F.Cu") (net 10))
 (segment (start 98.42 82.66) (end 99.255 82.66) (width 0.2) (layer "F.Cu") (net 18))
 (segment (start 89.0517 104.7737) (end 89.7784 105.5004) (width 0.2) (layer "F.Cu") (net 5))
 (segment (start 107.8947 105.5004) (end 108.918 106.5237) (width 0.2) (layer "F.Cu") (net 5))
 (segment (start 108.918 106.5237) (end 110.5287 106.5237) (width 0.2) (layer "F.Cu") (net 5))
 (segment (start 87.95 104.7737) (end 89.0517 104.7737) (width 0.2) (layer "F.Cu") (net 5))
 (segment (start 89.7784 105.5004) (end 107.8947 105.5004) (width 0.2) (layer "F.Cu") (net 5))
 (segment (start 108.9084 105.5517) (end 108.1304 104.7737) (width 0.2) (layer "F.Cu") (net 3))
 (segment (start 129.55 106.575) (end 128.4483 106.575) (width 0.2) (layer "F.Cu") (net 3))
 (segment (start 107.0287 104.7737) (end 108.1304 104.7737) (width 0.2) (layer "F.Cu") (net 3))
 (segment (start 127.425 105.5517) (end 108.9084 105.5517) (width 0.2) (layer "F.Cu") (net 3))
 (segment (start 128.4483 106.575) (end 127.425 105.5517) (width 0.2) (layer "F.Cu") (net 3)))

